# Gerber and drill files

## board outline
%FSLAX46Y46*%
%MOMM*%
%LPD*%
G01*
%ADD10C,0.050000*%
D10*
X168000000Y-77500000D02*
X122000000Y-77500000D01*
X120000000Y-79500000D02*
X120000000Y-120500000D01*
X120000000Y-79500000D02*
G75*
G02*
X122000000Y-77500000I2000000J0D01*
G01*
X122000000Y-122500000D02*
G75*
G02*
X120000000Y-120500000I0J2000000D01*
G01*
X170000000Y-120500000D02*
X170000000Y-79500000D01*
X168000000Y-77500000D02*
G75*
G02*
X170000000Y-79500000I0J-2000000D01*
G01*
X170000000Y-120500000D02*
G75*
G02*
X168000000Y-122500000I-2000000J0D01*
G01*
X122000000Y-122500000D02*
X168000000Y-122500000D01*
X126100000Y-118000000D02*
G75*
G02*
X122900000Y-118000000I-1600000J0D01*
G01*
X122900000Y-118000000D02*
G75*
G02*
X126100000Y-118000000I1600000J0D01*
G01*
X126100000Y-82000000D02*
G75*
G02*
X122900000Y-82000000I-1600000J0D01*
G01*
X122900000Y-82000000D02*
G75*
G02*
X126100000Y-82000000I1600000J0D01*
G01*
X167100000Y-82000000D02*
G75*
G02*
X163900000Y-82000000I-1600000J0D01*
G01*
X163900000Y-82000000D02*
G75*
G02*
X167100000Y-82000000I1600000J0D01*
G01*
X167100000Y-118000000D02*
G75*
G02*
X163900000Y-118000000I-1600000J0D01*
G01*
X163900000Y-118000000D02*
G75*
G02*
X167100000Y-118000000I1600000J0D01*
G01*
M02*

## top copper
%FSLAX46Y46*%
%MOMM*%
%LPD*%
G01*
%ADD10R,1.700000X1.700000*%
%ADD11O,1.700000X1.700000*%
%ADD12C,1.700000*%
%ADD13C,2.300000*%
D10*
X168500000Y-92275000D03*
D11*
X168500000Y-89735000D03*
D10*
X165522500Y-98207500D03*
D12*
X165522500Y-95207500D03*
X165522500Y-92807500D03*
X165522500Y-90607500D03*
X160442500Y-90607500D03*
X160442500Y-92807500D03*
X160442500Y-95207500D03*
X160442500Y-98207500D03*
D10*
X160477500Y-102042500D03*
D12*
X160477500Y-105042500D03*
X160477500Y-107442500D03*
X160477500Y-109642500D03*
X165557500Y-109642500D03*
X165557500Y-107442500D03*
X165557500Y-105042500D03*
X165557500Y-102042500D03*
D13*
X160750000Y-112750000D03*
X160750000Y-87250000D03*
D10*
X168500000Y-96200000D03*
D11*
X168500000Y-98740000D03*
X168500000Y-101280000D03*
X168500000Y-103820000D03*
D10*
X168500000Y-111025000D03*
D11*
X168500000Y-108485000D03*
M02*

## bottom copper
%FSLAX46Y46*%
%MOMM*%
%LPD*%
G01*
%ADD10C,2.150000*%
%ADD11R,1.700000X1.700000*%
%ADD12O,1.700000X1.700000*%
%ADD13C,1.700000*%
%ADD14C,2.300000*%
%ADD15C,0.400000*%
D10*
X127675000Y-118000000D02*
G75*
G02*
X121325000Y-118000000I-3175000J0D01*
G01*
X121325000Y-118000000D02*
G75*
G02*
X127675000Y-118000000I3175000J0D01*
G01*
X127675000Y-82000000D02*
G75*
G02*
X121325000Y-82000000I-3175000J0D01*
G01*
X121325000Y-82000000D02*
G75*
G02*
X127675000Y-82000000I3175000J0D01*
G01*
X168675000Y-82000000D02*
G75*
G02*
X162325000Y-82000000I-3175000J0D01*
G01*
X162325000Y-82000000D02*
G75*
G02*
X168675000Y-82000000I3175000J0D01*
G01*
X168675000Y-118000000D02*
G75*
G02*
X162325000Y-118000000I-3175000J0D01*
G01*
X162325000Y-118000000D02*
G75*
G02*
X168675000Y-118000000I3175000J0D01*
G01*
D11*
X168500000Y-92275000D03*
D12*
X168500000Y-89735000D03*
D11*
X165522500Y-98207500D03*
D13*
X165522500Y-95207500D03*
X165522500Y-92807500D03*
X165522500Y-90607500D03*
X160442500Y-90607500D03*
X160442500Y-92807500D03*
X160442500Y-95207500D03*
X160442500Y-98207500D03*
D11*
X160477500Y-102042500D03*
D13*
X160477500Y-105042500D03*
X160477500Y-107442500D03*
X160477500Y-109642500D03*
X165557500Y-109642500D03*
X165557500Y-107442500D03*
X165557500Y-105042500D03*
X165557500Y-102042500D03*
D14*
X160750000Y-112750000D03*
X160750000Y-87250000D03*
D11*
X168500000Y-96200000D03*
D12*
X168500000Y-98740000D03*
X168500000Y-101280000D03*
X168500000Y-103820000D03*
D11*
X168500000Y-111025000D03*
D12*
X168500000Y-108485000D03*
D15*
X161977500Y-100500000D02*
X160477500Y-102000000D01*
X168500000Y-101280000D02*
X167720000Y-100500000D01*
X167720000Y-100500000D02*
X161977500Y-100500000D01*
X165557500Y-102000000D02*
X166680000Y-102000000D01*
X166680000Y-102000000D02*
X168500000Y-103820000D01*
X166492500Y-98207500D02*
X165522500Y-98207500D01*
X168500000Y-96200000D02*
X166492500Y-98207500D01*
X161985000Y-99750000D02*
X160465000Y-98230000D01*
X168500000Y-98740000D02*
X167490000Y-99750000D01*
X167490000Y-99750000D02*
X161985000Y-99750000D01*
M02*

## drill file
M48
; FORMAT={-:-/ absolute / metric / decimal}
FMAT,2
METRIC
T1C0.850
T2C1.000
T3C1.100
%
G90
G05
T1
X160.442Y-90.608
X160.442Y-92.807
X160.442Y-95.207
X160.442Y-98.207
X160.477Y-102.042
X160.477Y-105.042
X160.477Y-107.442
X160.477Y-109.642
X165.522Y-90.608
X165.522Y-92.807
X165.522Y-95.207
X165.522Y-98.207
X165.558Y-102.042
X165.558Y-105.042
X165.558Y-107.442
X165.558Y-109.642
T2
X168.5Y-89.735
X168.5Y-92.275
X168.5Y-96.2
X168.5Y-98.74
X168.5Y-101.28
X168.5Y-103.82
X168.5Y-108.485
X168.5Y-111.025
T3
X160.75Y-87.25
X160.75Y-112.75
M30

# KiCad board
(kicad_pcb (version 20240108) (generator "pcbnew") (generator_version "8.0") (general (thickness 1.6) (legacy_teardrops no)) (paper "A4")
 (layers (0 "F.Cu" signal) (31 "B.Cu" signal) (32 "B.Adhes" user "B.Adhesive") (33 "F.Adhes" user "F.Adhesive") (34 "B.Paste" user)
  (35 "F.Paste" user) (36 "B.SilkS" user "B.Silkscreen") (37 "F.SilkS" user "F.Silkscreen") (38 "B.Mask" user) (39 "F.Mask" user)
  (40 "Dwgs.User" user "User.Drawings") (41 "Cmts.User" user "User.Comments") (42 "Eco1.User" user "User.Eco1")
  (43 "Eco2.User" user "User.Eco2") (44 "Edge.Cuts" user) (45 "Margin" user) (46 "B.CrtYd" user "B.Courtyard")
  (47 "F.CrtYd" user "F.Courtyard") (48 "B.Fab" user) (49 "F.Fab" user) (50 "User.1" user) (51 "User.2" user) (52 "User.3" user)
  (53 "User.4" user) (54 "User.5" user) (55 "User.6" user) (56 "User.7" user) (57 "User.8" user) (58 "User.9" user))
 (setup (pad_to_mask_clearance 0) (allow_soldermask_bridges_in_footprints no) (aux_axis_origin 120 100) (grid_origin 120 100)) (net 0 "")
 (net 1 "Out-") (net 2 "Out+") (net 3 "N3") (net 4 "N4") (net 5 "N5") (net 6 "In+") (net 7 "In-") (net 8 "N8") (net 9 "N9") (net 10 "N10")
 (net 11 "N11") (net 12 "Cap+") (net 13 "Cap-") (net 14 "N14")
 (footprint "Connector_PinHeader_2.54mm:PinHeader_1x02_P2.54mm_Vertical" (layer "F.Cu") (at 168.5 92.275 180)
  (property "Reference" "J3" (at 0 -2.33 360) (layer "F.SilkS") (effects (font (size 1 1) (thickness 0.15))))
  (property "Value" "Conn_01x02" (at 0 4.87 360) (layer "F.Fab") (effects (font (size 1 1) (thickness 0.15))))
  (pad "1" thru_hole rect (at 0 0 180) (size 1.7 1.7) (drill 1) (layers "*.Cu" "*.Mask") (remove_unused_layers no) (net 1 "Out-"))
  (pad "2" thru_hole oval (at 0 2.54 180) (size 1.7 1.7) (drill 1) (layers "*.Cu" "*.Mask") (remove_unused_layers no) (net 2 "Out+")))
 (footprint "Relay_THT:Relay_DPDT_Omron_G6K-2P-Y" (layer "F.Cu") (at 165.5225 98.2075 180)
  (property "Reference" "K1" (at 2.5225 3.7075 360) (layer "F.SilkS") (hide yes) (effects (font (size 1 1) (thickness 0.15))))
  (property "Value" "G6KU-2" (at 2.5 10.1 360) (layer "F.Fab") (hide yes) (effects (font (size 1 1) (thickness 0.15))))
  (pad "1" thru_hole rect (at 0 0 180) (size 1.7 1.7) (drill 0.85) (layers "*.Cu" "*.Mask") (remove_unused_layers no) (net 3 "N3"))
  (pad "2" thru_hole circle (at 0 3 180) (size 1.7 1.7) (drill 0.85) (layers "*.Cu" "*.Mask") (remove_unused_layers no) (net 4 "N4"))
  (pad "3" thru_hole circle (at 0 5.4 180) (size 1.7 1.7) (drill 0.85) (layers "*.Cu" "*.Mask") (remove_unused_layers no) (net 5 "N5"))
  (pad "4" thru_hole circle (at 0 7.6 180) (size 1.7 1.7) (drill 0.85) (layers "*.Cu" "*.Mask") (remove_unused_layers no) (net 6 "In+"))
  (pad "5" thru_hole circle (at 5.08 7.6 180) (size 1.7 1.7) (drill 0.85) (layers "*.Cu" "*.Mask") (remove_unused_layers no) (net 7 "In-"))
  (pad "6" thru_hole circle (at 5.08 5.4 180) (size 1.7 1.7) (drill 0.85) (layers "*.Cu" "*.Mask") (remove_unused_layers no) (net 1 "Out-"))
  (pad "7" thru_hole circle (at 5.08 3 180) (size 1.7 1.7) (drill 0.85) (layers "*.Cu" "*.Mask") (remove_unused_layers no) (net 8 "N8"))
  (pad "8" thru_hole circle (at 5.08 0 180) (size 1.7 1.7) (drill 0.85) (layers "*.Cu" "*.Mask") (remove_unused_layers no) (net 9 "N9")))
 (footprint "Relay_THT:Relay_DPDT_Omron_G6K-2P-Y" (layer "F.Cu") (at 160.4775 102.0425)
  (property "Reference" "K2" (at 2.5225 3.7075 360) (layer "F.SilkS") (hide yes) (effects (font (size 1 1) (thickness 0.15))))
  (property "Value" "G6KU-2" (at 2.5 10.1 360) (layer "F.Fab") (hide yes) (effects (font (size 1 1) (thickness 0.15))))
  (pad "1" thru_hole rect (at 0 0) (size 1.7 1.7) (drill 0.85) (layers "*.Cu" "*.Mask") (remove_unused_layers no) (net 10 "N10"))
  (pad "2" thru_hole circle (at 0 3) (size 1.7 1.7) (drill 0.85) (layers "*.Cu" "*.Mask") (remove_unused_layers no) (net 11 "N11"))
  (pad "3" thru_hole circle (at 0 5.4) (size 1.7 1.7) (drill 0.85) (layers "*.Cu" "*.Mask") (remove_unused_layers no) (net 5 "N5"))
  (pad "4" thru_hole circle (at 0 7.6) (size 1.7 1.7) (drill 0.85) (layers "*.Cu" "*.Mask") (remove_unused_layers no) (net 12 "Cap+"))
  (pad "5" thru_hole circle (at 5.08 7.6) (size 1.7 1.7) (drill 0.85) (layers "*.Cu" "*.Mask") (remove_unused_layers no) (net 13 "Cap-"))
  (pad "6" thru_hole circle (at 5.08 5.4) (size 1.7 1.7) (drill 0.85) (layers "*.Cu" "*.Mask") (remove_unused_layers no) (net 2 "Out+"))
  (pad "7" thru_hole circle (at 5.08 3) (size 1.7 1.7) (drill 0.85) (layers "*.Cu" "*.Mask") (remove_unused_layers no) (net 11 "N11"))
  (pad "8" thru_hole circle (at 5.08 0) (size 1.7 1.7) (drill 0.85) (layers "*.Cu" "*.Mask") (remove_unused_layers no) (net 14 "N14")))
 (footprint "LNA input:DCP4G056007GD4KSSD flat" (layer "F.Cu") (at 121.75 100)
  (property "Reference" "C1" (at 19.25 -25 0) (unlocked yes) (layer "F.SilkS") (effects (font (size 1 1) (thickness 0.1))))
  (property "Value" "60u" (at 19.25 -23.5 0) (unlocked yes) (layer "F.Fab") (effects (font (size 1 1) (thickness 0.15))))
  (pad "1" thru_hole circle (at 39 12.75) (size 2.3 2.3) (drill 1.1) (layers "*.Cu" "*.Mask") (remove_unused_layers no) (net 13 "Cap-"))
  (pad "2" thru_hole circle (at 39 -12.75) (size 2.3 2.3) (drill 1.1) (layers "*.Cu" "*.Mask") (remove_unused_layers no) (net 12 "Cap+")))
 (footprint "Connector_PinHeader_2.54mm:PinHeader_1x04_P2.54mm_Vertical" (layer "F.Cu") (at 168.5 96.2)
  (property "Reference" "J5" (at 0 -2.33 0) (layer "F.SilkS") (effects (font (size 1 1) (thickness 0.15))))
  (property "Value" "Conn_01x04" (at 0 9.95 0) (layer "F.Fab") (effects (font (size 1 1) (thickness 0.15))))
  (pad "1" thru_hole rect (at 0 0) (size 1.7 1.7) (drill 1) (layers "*.Cu" "*.Mask") (remove_unused_layers no) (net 3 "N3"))
  (pad "2" thru_hole oval (at 0 2.54) (size 1.7 1.7) (drill 1) (layers "*.Cu" "*.Mask") (remove_unused_layers no) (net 9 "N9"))
  (pad "3" thru_hole oval (at 0 5.08) (size 1.7 1.7) (drill 1) (layers "*.Cu" "*.Mask") (remove_unused_layers no) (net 10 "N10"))
  (pad "4" thru_hole oval (at 0 7.62) (size 1.7 1.7) (drill 1) (layers "*.Cu" "*.Mask") (remove_unused_layers no) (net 14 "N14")))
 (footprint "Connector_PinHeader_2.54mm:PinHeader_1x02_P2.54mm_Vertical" (layer "F.Cu") (at 168.5 111.025 180)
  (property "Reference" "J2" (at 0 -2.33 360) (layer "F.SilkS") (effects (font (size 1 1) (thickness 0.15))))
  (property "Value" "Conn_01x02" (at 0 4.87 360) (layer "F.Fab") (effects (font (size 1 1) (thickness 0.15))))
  (pad "1" thru_hole rect (at 0 0 180) (size 1.7 1.7) (drill 1) (layers "*.Cu" "*.Mask") (remove_unused_layers no) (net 6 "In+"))
  (pad "2" thru_hole oval (at 0 2.54 180) (size 1.7 1.7) (drill 1) (layers "*.Cu" "*.Mask") (remove_unused_layers no) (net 7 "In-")))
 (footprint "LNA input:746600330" (layer "B.Cu") (at 124.5 118 180)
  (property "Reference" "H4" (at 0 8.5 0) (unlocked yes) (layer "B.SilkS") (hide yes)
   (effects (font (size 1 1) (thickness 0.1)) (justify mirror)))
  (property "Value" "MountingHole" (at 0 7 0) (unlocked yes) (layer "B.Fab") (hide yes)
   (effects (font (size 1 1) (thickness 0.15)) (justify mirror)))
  (fp_circle (center 0 0) (end 3.175 0) (stroke (width 2.15) (type default)) (fill none) (layer "B.Cu"))
  (fp_circle (center 0 0) (end 1.6 0) (stroke (width 0.05) (type default)) (fill none) (layer "Edge.Cuts")))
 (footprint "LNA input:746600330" (layer "B.Cu") (at 124.5 82 180)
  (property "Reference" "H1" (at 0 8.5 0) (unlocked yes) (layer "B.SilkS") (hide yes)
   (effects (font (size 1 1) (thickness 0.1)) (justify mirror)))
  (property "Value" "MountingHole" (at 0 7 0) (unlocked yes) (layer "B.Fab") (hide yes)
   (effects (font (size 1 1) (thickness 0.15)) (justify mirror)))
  (fp_circle (center 0 0) (end 3.175 0) (stroke (width 2.15) (type default)) (fill none) (layer "B.Cu"))
  (fp_circle (center 0 0) (end 1.6 0) (stroke (width 0.05) (type default)) (fill none) (layer "Edge.Cuts")))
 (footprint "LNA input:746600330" (layer "B.Cu") (at 165.5 82 180)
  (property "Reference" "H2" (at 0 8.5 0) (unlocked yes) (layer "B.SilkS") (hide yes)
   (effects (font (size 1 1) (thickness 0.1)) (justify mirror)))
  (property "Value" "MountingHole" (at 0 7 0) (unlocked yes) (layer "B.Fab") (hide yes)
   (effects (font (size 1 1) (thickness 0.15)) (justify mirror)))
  (fp_circle (center 0 0) (end 3.175 0) (stroke (width 2.15) (type default)) (fill none) (layer "B.Cu"))
  (fp_circle (center 0 0) (end 1.6 0) (stroke (width 0.05) (type default)) (fill none) (layer "Edge.Cuts")))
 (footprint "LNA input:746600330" (layer "B.Cu") (at 165.5 118 180)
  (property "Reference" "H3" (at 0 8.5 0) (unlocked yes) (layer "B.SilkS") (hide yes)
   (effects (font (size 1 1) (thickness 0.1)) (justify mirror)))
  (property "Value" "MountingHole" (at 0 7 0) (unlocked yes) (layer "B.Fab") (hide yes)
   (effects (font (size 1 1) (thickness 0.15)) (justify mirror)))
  (fp_circle (center 0 0) (end 3.175 0) (stroke (width 2.15) (type default)) (fill none) (layer "B.Cu"))
  (fp_circle (center 0 0) (end 1.6 0) (stroke (width 0.05) (type default)) (fill none) (layer "Edge.Cuts")))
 (gr_line (start 168 77.5) (end 122 77.5) (stroke (width 0.05) (type default)) (layer "Edge.Cuts"))
 (gr_line (start 120 79.5) (end 120 120.5) (stroke (width 0.05) (type default)) (layer "Edge.Cuts"))
 (gr_arc (start 120 79.5) (mid 120.585786 78.085786) (end 122 77.5) (stroke (width 0.05) (type default)) (layer "Edge.Cuts"))
 (gr_arc (start 122 122.5) (mid 120.585786 121.914214) (end 120 120.5) (stroke (width 0.05) (type default)) (layer "Edge.Cuts"))
 (gr_line (start 170 120.5) (end 170 79.5) (stroke (width 0.05) (type default)) (layer "Edge.Cuts"))
 (gr_arc (start 168 77.5) (mid 169.414214 78.085786) (end 170 79.5) (stroke (width 0.05) (type default)) (layer "Edge.Cuts"))
 (gr_arc (start 170 120.5) (mid 169.414214 121.914214) (end 168 122.5) (stroke (width 0.05) (type default)) (layer "Edge.Cuts"))
 (gr_line (start 122 122.5) (end 168 122.5) (stroke (width 0.05) (type default)) (layer "Edge.Cuts"))
 (segment (start 161.9775 100.5) (end 160.4775 102) (width 0.4) (layer "B.Cu") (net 10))
 (segment (start 168.5 101.28) (end 167.72 100.5) (width 0.4) (layer "B.Cu") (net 10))
 (segment (start 167.72 100.5) (end 161.9775 100.5) (width 0.4) (layer "B.Cu") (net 10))
 (segment (start 165.5575 102) (end 166.68 102) (width 0.4) (layer "B.Cu") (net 14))
 (segment (start 166.68 102) (end 168.5 103.82) (width 0.4) (layer "B.Cu") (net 14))
 (segment (start 166.4925 98.2075) (end 165.5225 98.2075) (width 0.4) (layer "B.Cu") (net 3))
 (segment (start 168.5 96.2) (end 166.4925 98.2075) (width 0.4) (layer "B.Cu") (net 3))
 (segment (start 161.985 99.75) (end 160.465 98.23) (width 0.4) (layer "B.Cu") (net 9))
 (segment (start 168.5 98.74) (end 167.49 99.75) (width 0.4) (layer "B.Cu") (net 9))
 (segment (start 167.49 99.75) (end 161.985 99.75) (width 0.4) (layer "B.Cu") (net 9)))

